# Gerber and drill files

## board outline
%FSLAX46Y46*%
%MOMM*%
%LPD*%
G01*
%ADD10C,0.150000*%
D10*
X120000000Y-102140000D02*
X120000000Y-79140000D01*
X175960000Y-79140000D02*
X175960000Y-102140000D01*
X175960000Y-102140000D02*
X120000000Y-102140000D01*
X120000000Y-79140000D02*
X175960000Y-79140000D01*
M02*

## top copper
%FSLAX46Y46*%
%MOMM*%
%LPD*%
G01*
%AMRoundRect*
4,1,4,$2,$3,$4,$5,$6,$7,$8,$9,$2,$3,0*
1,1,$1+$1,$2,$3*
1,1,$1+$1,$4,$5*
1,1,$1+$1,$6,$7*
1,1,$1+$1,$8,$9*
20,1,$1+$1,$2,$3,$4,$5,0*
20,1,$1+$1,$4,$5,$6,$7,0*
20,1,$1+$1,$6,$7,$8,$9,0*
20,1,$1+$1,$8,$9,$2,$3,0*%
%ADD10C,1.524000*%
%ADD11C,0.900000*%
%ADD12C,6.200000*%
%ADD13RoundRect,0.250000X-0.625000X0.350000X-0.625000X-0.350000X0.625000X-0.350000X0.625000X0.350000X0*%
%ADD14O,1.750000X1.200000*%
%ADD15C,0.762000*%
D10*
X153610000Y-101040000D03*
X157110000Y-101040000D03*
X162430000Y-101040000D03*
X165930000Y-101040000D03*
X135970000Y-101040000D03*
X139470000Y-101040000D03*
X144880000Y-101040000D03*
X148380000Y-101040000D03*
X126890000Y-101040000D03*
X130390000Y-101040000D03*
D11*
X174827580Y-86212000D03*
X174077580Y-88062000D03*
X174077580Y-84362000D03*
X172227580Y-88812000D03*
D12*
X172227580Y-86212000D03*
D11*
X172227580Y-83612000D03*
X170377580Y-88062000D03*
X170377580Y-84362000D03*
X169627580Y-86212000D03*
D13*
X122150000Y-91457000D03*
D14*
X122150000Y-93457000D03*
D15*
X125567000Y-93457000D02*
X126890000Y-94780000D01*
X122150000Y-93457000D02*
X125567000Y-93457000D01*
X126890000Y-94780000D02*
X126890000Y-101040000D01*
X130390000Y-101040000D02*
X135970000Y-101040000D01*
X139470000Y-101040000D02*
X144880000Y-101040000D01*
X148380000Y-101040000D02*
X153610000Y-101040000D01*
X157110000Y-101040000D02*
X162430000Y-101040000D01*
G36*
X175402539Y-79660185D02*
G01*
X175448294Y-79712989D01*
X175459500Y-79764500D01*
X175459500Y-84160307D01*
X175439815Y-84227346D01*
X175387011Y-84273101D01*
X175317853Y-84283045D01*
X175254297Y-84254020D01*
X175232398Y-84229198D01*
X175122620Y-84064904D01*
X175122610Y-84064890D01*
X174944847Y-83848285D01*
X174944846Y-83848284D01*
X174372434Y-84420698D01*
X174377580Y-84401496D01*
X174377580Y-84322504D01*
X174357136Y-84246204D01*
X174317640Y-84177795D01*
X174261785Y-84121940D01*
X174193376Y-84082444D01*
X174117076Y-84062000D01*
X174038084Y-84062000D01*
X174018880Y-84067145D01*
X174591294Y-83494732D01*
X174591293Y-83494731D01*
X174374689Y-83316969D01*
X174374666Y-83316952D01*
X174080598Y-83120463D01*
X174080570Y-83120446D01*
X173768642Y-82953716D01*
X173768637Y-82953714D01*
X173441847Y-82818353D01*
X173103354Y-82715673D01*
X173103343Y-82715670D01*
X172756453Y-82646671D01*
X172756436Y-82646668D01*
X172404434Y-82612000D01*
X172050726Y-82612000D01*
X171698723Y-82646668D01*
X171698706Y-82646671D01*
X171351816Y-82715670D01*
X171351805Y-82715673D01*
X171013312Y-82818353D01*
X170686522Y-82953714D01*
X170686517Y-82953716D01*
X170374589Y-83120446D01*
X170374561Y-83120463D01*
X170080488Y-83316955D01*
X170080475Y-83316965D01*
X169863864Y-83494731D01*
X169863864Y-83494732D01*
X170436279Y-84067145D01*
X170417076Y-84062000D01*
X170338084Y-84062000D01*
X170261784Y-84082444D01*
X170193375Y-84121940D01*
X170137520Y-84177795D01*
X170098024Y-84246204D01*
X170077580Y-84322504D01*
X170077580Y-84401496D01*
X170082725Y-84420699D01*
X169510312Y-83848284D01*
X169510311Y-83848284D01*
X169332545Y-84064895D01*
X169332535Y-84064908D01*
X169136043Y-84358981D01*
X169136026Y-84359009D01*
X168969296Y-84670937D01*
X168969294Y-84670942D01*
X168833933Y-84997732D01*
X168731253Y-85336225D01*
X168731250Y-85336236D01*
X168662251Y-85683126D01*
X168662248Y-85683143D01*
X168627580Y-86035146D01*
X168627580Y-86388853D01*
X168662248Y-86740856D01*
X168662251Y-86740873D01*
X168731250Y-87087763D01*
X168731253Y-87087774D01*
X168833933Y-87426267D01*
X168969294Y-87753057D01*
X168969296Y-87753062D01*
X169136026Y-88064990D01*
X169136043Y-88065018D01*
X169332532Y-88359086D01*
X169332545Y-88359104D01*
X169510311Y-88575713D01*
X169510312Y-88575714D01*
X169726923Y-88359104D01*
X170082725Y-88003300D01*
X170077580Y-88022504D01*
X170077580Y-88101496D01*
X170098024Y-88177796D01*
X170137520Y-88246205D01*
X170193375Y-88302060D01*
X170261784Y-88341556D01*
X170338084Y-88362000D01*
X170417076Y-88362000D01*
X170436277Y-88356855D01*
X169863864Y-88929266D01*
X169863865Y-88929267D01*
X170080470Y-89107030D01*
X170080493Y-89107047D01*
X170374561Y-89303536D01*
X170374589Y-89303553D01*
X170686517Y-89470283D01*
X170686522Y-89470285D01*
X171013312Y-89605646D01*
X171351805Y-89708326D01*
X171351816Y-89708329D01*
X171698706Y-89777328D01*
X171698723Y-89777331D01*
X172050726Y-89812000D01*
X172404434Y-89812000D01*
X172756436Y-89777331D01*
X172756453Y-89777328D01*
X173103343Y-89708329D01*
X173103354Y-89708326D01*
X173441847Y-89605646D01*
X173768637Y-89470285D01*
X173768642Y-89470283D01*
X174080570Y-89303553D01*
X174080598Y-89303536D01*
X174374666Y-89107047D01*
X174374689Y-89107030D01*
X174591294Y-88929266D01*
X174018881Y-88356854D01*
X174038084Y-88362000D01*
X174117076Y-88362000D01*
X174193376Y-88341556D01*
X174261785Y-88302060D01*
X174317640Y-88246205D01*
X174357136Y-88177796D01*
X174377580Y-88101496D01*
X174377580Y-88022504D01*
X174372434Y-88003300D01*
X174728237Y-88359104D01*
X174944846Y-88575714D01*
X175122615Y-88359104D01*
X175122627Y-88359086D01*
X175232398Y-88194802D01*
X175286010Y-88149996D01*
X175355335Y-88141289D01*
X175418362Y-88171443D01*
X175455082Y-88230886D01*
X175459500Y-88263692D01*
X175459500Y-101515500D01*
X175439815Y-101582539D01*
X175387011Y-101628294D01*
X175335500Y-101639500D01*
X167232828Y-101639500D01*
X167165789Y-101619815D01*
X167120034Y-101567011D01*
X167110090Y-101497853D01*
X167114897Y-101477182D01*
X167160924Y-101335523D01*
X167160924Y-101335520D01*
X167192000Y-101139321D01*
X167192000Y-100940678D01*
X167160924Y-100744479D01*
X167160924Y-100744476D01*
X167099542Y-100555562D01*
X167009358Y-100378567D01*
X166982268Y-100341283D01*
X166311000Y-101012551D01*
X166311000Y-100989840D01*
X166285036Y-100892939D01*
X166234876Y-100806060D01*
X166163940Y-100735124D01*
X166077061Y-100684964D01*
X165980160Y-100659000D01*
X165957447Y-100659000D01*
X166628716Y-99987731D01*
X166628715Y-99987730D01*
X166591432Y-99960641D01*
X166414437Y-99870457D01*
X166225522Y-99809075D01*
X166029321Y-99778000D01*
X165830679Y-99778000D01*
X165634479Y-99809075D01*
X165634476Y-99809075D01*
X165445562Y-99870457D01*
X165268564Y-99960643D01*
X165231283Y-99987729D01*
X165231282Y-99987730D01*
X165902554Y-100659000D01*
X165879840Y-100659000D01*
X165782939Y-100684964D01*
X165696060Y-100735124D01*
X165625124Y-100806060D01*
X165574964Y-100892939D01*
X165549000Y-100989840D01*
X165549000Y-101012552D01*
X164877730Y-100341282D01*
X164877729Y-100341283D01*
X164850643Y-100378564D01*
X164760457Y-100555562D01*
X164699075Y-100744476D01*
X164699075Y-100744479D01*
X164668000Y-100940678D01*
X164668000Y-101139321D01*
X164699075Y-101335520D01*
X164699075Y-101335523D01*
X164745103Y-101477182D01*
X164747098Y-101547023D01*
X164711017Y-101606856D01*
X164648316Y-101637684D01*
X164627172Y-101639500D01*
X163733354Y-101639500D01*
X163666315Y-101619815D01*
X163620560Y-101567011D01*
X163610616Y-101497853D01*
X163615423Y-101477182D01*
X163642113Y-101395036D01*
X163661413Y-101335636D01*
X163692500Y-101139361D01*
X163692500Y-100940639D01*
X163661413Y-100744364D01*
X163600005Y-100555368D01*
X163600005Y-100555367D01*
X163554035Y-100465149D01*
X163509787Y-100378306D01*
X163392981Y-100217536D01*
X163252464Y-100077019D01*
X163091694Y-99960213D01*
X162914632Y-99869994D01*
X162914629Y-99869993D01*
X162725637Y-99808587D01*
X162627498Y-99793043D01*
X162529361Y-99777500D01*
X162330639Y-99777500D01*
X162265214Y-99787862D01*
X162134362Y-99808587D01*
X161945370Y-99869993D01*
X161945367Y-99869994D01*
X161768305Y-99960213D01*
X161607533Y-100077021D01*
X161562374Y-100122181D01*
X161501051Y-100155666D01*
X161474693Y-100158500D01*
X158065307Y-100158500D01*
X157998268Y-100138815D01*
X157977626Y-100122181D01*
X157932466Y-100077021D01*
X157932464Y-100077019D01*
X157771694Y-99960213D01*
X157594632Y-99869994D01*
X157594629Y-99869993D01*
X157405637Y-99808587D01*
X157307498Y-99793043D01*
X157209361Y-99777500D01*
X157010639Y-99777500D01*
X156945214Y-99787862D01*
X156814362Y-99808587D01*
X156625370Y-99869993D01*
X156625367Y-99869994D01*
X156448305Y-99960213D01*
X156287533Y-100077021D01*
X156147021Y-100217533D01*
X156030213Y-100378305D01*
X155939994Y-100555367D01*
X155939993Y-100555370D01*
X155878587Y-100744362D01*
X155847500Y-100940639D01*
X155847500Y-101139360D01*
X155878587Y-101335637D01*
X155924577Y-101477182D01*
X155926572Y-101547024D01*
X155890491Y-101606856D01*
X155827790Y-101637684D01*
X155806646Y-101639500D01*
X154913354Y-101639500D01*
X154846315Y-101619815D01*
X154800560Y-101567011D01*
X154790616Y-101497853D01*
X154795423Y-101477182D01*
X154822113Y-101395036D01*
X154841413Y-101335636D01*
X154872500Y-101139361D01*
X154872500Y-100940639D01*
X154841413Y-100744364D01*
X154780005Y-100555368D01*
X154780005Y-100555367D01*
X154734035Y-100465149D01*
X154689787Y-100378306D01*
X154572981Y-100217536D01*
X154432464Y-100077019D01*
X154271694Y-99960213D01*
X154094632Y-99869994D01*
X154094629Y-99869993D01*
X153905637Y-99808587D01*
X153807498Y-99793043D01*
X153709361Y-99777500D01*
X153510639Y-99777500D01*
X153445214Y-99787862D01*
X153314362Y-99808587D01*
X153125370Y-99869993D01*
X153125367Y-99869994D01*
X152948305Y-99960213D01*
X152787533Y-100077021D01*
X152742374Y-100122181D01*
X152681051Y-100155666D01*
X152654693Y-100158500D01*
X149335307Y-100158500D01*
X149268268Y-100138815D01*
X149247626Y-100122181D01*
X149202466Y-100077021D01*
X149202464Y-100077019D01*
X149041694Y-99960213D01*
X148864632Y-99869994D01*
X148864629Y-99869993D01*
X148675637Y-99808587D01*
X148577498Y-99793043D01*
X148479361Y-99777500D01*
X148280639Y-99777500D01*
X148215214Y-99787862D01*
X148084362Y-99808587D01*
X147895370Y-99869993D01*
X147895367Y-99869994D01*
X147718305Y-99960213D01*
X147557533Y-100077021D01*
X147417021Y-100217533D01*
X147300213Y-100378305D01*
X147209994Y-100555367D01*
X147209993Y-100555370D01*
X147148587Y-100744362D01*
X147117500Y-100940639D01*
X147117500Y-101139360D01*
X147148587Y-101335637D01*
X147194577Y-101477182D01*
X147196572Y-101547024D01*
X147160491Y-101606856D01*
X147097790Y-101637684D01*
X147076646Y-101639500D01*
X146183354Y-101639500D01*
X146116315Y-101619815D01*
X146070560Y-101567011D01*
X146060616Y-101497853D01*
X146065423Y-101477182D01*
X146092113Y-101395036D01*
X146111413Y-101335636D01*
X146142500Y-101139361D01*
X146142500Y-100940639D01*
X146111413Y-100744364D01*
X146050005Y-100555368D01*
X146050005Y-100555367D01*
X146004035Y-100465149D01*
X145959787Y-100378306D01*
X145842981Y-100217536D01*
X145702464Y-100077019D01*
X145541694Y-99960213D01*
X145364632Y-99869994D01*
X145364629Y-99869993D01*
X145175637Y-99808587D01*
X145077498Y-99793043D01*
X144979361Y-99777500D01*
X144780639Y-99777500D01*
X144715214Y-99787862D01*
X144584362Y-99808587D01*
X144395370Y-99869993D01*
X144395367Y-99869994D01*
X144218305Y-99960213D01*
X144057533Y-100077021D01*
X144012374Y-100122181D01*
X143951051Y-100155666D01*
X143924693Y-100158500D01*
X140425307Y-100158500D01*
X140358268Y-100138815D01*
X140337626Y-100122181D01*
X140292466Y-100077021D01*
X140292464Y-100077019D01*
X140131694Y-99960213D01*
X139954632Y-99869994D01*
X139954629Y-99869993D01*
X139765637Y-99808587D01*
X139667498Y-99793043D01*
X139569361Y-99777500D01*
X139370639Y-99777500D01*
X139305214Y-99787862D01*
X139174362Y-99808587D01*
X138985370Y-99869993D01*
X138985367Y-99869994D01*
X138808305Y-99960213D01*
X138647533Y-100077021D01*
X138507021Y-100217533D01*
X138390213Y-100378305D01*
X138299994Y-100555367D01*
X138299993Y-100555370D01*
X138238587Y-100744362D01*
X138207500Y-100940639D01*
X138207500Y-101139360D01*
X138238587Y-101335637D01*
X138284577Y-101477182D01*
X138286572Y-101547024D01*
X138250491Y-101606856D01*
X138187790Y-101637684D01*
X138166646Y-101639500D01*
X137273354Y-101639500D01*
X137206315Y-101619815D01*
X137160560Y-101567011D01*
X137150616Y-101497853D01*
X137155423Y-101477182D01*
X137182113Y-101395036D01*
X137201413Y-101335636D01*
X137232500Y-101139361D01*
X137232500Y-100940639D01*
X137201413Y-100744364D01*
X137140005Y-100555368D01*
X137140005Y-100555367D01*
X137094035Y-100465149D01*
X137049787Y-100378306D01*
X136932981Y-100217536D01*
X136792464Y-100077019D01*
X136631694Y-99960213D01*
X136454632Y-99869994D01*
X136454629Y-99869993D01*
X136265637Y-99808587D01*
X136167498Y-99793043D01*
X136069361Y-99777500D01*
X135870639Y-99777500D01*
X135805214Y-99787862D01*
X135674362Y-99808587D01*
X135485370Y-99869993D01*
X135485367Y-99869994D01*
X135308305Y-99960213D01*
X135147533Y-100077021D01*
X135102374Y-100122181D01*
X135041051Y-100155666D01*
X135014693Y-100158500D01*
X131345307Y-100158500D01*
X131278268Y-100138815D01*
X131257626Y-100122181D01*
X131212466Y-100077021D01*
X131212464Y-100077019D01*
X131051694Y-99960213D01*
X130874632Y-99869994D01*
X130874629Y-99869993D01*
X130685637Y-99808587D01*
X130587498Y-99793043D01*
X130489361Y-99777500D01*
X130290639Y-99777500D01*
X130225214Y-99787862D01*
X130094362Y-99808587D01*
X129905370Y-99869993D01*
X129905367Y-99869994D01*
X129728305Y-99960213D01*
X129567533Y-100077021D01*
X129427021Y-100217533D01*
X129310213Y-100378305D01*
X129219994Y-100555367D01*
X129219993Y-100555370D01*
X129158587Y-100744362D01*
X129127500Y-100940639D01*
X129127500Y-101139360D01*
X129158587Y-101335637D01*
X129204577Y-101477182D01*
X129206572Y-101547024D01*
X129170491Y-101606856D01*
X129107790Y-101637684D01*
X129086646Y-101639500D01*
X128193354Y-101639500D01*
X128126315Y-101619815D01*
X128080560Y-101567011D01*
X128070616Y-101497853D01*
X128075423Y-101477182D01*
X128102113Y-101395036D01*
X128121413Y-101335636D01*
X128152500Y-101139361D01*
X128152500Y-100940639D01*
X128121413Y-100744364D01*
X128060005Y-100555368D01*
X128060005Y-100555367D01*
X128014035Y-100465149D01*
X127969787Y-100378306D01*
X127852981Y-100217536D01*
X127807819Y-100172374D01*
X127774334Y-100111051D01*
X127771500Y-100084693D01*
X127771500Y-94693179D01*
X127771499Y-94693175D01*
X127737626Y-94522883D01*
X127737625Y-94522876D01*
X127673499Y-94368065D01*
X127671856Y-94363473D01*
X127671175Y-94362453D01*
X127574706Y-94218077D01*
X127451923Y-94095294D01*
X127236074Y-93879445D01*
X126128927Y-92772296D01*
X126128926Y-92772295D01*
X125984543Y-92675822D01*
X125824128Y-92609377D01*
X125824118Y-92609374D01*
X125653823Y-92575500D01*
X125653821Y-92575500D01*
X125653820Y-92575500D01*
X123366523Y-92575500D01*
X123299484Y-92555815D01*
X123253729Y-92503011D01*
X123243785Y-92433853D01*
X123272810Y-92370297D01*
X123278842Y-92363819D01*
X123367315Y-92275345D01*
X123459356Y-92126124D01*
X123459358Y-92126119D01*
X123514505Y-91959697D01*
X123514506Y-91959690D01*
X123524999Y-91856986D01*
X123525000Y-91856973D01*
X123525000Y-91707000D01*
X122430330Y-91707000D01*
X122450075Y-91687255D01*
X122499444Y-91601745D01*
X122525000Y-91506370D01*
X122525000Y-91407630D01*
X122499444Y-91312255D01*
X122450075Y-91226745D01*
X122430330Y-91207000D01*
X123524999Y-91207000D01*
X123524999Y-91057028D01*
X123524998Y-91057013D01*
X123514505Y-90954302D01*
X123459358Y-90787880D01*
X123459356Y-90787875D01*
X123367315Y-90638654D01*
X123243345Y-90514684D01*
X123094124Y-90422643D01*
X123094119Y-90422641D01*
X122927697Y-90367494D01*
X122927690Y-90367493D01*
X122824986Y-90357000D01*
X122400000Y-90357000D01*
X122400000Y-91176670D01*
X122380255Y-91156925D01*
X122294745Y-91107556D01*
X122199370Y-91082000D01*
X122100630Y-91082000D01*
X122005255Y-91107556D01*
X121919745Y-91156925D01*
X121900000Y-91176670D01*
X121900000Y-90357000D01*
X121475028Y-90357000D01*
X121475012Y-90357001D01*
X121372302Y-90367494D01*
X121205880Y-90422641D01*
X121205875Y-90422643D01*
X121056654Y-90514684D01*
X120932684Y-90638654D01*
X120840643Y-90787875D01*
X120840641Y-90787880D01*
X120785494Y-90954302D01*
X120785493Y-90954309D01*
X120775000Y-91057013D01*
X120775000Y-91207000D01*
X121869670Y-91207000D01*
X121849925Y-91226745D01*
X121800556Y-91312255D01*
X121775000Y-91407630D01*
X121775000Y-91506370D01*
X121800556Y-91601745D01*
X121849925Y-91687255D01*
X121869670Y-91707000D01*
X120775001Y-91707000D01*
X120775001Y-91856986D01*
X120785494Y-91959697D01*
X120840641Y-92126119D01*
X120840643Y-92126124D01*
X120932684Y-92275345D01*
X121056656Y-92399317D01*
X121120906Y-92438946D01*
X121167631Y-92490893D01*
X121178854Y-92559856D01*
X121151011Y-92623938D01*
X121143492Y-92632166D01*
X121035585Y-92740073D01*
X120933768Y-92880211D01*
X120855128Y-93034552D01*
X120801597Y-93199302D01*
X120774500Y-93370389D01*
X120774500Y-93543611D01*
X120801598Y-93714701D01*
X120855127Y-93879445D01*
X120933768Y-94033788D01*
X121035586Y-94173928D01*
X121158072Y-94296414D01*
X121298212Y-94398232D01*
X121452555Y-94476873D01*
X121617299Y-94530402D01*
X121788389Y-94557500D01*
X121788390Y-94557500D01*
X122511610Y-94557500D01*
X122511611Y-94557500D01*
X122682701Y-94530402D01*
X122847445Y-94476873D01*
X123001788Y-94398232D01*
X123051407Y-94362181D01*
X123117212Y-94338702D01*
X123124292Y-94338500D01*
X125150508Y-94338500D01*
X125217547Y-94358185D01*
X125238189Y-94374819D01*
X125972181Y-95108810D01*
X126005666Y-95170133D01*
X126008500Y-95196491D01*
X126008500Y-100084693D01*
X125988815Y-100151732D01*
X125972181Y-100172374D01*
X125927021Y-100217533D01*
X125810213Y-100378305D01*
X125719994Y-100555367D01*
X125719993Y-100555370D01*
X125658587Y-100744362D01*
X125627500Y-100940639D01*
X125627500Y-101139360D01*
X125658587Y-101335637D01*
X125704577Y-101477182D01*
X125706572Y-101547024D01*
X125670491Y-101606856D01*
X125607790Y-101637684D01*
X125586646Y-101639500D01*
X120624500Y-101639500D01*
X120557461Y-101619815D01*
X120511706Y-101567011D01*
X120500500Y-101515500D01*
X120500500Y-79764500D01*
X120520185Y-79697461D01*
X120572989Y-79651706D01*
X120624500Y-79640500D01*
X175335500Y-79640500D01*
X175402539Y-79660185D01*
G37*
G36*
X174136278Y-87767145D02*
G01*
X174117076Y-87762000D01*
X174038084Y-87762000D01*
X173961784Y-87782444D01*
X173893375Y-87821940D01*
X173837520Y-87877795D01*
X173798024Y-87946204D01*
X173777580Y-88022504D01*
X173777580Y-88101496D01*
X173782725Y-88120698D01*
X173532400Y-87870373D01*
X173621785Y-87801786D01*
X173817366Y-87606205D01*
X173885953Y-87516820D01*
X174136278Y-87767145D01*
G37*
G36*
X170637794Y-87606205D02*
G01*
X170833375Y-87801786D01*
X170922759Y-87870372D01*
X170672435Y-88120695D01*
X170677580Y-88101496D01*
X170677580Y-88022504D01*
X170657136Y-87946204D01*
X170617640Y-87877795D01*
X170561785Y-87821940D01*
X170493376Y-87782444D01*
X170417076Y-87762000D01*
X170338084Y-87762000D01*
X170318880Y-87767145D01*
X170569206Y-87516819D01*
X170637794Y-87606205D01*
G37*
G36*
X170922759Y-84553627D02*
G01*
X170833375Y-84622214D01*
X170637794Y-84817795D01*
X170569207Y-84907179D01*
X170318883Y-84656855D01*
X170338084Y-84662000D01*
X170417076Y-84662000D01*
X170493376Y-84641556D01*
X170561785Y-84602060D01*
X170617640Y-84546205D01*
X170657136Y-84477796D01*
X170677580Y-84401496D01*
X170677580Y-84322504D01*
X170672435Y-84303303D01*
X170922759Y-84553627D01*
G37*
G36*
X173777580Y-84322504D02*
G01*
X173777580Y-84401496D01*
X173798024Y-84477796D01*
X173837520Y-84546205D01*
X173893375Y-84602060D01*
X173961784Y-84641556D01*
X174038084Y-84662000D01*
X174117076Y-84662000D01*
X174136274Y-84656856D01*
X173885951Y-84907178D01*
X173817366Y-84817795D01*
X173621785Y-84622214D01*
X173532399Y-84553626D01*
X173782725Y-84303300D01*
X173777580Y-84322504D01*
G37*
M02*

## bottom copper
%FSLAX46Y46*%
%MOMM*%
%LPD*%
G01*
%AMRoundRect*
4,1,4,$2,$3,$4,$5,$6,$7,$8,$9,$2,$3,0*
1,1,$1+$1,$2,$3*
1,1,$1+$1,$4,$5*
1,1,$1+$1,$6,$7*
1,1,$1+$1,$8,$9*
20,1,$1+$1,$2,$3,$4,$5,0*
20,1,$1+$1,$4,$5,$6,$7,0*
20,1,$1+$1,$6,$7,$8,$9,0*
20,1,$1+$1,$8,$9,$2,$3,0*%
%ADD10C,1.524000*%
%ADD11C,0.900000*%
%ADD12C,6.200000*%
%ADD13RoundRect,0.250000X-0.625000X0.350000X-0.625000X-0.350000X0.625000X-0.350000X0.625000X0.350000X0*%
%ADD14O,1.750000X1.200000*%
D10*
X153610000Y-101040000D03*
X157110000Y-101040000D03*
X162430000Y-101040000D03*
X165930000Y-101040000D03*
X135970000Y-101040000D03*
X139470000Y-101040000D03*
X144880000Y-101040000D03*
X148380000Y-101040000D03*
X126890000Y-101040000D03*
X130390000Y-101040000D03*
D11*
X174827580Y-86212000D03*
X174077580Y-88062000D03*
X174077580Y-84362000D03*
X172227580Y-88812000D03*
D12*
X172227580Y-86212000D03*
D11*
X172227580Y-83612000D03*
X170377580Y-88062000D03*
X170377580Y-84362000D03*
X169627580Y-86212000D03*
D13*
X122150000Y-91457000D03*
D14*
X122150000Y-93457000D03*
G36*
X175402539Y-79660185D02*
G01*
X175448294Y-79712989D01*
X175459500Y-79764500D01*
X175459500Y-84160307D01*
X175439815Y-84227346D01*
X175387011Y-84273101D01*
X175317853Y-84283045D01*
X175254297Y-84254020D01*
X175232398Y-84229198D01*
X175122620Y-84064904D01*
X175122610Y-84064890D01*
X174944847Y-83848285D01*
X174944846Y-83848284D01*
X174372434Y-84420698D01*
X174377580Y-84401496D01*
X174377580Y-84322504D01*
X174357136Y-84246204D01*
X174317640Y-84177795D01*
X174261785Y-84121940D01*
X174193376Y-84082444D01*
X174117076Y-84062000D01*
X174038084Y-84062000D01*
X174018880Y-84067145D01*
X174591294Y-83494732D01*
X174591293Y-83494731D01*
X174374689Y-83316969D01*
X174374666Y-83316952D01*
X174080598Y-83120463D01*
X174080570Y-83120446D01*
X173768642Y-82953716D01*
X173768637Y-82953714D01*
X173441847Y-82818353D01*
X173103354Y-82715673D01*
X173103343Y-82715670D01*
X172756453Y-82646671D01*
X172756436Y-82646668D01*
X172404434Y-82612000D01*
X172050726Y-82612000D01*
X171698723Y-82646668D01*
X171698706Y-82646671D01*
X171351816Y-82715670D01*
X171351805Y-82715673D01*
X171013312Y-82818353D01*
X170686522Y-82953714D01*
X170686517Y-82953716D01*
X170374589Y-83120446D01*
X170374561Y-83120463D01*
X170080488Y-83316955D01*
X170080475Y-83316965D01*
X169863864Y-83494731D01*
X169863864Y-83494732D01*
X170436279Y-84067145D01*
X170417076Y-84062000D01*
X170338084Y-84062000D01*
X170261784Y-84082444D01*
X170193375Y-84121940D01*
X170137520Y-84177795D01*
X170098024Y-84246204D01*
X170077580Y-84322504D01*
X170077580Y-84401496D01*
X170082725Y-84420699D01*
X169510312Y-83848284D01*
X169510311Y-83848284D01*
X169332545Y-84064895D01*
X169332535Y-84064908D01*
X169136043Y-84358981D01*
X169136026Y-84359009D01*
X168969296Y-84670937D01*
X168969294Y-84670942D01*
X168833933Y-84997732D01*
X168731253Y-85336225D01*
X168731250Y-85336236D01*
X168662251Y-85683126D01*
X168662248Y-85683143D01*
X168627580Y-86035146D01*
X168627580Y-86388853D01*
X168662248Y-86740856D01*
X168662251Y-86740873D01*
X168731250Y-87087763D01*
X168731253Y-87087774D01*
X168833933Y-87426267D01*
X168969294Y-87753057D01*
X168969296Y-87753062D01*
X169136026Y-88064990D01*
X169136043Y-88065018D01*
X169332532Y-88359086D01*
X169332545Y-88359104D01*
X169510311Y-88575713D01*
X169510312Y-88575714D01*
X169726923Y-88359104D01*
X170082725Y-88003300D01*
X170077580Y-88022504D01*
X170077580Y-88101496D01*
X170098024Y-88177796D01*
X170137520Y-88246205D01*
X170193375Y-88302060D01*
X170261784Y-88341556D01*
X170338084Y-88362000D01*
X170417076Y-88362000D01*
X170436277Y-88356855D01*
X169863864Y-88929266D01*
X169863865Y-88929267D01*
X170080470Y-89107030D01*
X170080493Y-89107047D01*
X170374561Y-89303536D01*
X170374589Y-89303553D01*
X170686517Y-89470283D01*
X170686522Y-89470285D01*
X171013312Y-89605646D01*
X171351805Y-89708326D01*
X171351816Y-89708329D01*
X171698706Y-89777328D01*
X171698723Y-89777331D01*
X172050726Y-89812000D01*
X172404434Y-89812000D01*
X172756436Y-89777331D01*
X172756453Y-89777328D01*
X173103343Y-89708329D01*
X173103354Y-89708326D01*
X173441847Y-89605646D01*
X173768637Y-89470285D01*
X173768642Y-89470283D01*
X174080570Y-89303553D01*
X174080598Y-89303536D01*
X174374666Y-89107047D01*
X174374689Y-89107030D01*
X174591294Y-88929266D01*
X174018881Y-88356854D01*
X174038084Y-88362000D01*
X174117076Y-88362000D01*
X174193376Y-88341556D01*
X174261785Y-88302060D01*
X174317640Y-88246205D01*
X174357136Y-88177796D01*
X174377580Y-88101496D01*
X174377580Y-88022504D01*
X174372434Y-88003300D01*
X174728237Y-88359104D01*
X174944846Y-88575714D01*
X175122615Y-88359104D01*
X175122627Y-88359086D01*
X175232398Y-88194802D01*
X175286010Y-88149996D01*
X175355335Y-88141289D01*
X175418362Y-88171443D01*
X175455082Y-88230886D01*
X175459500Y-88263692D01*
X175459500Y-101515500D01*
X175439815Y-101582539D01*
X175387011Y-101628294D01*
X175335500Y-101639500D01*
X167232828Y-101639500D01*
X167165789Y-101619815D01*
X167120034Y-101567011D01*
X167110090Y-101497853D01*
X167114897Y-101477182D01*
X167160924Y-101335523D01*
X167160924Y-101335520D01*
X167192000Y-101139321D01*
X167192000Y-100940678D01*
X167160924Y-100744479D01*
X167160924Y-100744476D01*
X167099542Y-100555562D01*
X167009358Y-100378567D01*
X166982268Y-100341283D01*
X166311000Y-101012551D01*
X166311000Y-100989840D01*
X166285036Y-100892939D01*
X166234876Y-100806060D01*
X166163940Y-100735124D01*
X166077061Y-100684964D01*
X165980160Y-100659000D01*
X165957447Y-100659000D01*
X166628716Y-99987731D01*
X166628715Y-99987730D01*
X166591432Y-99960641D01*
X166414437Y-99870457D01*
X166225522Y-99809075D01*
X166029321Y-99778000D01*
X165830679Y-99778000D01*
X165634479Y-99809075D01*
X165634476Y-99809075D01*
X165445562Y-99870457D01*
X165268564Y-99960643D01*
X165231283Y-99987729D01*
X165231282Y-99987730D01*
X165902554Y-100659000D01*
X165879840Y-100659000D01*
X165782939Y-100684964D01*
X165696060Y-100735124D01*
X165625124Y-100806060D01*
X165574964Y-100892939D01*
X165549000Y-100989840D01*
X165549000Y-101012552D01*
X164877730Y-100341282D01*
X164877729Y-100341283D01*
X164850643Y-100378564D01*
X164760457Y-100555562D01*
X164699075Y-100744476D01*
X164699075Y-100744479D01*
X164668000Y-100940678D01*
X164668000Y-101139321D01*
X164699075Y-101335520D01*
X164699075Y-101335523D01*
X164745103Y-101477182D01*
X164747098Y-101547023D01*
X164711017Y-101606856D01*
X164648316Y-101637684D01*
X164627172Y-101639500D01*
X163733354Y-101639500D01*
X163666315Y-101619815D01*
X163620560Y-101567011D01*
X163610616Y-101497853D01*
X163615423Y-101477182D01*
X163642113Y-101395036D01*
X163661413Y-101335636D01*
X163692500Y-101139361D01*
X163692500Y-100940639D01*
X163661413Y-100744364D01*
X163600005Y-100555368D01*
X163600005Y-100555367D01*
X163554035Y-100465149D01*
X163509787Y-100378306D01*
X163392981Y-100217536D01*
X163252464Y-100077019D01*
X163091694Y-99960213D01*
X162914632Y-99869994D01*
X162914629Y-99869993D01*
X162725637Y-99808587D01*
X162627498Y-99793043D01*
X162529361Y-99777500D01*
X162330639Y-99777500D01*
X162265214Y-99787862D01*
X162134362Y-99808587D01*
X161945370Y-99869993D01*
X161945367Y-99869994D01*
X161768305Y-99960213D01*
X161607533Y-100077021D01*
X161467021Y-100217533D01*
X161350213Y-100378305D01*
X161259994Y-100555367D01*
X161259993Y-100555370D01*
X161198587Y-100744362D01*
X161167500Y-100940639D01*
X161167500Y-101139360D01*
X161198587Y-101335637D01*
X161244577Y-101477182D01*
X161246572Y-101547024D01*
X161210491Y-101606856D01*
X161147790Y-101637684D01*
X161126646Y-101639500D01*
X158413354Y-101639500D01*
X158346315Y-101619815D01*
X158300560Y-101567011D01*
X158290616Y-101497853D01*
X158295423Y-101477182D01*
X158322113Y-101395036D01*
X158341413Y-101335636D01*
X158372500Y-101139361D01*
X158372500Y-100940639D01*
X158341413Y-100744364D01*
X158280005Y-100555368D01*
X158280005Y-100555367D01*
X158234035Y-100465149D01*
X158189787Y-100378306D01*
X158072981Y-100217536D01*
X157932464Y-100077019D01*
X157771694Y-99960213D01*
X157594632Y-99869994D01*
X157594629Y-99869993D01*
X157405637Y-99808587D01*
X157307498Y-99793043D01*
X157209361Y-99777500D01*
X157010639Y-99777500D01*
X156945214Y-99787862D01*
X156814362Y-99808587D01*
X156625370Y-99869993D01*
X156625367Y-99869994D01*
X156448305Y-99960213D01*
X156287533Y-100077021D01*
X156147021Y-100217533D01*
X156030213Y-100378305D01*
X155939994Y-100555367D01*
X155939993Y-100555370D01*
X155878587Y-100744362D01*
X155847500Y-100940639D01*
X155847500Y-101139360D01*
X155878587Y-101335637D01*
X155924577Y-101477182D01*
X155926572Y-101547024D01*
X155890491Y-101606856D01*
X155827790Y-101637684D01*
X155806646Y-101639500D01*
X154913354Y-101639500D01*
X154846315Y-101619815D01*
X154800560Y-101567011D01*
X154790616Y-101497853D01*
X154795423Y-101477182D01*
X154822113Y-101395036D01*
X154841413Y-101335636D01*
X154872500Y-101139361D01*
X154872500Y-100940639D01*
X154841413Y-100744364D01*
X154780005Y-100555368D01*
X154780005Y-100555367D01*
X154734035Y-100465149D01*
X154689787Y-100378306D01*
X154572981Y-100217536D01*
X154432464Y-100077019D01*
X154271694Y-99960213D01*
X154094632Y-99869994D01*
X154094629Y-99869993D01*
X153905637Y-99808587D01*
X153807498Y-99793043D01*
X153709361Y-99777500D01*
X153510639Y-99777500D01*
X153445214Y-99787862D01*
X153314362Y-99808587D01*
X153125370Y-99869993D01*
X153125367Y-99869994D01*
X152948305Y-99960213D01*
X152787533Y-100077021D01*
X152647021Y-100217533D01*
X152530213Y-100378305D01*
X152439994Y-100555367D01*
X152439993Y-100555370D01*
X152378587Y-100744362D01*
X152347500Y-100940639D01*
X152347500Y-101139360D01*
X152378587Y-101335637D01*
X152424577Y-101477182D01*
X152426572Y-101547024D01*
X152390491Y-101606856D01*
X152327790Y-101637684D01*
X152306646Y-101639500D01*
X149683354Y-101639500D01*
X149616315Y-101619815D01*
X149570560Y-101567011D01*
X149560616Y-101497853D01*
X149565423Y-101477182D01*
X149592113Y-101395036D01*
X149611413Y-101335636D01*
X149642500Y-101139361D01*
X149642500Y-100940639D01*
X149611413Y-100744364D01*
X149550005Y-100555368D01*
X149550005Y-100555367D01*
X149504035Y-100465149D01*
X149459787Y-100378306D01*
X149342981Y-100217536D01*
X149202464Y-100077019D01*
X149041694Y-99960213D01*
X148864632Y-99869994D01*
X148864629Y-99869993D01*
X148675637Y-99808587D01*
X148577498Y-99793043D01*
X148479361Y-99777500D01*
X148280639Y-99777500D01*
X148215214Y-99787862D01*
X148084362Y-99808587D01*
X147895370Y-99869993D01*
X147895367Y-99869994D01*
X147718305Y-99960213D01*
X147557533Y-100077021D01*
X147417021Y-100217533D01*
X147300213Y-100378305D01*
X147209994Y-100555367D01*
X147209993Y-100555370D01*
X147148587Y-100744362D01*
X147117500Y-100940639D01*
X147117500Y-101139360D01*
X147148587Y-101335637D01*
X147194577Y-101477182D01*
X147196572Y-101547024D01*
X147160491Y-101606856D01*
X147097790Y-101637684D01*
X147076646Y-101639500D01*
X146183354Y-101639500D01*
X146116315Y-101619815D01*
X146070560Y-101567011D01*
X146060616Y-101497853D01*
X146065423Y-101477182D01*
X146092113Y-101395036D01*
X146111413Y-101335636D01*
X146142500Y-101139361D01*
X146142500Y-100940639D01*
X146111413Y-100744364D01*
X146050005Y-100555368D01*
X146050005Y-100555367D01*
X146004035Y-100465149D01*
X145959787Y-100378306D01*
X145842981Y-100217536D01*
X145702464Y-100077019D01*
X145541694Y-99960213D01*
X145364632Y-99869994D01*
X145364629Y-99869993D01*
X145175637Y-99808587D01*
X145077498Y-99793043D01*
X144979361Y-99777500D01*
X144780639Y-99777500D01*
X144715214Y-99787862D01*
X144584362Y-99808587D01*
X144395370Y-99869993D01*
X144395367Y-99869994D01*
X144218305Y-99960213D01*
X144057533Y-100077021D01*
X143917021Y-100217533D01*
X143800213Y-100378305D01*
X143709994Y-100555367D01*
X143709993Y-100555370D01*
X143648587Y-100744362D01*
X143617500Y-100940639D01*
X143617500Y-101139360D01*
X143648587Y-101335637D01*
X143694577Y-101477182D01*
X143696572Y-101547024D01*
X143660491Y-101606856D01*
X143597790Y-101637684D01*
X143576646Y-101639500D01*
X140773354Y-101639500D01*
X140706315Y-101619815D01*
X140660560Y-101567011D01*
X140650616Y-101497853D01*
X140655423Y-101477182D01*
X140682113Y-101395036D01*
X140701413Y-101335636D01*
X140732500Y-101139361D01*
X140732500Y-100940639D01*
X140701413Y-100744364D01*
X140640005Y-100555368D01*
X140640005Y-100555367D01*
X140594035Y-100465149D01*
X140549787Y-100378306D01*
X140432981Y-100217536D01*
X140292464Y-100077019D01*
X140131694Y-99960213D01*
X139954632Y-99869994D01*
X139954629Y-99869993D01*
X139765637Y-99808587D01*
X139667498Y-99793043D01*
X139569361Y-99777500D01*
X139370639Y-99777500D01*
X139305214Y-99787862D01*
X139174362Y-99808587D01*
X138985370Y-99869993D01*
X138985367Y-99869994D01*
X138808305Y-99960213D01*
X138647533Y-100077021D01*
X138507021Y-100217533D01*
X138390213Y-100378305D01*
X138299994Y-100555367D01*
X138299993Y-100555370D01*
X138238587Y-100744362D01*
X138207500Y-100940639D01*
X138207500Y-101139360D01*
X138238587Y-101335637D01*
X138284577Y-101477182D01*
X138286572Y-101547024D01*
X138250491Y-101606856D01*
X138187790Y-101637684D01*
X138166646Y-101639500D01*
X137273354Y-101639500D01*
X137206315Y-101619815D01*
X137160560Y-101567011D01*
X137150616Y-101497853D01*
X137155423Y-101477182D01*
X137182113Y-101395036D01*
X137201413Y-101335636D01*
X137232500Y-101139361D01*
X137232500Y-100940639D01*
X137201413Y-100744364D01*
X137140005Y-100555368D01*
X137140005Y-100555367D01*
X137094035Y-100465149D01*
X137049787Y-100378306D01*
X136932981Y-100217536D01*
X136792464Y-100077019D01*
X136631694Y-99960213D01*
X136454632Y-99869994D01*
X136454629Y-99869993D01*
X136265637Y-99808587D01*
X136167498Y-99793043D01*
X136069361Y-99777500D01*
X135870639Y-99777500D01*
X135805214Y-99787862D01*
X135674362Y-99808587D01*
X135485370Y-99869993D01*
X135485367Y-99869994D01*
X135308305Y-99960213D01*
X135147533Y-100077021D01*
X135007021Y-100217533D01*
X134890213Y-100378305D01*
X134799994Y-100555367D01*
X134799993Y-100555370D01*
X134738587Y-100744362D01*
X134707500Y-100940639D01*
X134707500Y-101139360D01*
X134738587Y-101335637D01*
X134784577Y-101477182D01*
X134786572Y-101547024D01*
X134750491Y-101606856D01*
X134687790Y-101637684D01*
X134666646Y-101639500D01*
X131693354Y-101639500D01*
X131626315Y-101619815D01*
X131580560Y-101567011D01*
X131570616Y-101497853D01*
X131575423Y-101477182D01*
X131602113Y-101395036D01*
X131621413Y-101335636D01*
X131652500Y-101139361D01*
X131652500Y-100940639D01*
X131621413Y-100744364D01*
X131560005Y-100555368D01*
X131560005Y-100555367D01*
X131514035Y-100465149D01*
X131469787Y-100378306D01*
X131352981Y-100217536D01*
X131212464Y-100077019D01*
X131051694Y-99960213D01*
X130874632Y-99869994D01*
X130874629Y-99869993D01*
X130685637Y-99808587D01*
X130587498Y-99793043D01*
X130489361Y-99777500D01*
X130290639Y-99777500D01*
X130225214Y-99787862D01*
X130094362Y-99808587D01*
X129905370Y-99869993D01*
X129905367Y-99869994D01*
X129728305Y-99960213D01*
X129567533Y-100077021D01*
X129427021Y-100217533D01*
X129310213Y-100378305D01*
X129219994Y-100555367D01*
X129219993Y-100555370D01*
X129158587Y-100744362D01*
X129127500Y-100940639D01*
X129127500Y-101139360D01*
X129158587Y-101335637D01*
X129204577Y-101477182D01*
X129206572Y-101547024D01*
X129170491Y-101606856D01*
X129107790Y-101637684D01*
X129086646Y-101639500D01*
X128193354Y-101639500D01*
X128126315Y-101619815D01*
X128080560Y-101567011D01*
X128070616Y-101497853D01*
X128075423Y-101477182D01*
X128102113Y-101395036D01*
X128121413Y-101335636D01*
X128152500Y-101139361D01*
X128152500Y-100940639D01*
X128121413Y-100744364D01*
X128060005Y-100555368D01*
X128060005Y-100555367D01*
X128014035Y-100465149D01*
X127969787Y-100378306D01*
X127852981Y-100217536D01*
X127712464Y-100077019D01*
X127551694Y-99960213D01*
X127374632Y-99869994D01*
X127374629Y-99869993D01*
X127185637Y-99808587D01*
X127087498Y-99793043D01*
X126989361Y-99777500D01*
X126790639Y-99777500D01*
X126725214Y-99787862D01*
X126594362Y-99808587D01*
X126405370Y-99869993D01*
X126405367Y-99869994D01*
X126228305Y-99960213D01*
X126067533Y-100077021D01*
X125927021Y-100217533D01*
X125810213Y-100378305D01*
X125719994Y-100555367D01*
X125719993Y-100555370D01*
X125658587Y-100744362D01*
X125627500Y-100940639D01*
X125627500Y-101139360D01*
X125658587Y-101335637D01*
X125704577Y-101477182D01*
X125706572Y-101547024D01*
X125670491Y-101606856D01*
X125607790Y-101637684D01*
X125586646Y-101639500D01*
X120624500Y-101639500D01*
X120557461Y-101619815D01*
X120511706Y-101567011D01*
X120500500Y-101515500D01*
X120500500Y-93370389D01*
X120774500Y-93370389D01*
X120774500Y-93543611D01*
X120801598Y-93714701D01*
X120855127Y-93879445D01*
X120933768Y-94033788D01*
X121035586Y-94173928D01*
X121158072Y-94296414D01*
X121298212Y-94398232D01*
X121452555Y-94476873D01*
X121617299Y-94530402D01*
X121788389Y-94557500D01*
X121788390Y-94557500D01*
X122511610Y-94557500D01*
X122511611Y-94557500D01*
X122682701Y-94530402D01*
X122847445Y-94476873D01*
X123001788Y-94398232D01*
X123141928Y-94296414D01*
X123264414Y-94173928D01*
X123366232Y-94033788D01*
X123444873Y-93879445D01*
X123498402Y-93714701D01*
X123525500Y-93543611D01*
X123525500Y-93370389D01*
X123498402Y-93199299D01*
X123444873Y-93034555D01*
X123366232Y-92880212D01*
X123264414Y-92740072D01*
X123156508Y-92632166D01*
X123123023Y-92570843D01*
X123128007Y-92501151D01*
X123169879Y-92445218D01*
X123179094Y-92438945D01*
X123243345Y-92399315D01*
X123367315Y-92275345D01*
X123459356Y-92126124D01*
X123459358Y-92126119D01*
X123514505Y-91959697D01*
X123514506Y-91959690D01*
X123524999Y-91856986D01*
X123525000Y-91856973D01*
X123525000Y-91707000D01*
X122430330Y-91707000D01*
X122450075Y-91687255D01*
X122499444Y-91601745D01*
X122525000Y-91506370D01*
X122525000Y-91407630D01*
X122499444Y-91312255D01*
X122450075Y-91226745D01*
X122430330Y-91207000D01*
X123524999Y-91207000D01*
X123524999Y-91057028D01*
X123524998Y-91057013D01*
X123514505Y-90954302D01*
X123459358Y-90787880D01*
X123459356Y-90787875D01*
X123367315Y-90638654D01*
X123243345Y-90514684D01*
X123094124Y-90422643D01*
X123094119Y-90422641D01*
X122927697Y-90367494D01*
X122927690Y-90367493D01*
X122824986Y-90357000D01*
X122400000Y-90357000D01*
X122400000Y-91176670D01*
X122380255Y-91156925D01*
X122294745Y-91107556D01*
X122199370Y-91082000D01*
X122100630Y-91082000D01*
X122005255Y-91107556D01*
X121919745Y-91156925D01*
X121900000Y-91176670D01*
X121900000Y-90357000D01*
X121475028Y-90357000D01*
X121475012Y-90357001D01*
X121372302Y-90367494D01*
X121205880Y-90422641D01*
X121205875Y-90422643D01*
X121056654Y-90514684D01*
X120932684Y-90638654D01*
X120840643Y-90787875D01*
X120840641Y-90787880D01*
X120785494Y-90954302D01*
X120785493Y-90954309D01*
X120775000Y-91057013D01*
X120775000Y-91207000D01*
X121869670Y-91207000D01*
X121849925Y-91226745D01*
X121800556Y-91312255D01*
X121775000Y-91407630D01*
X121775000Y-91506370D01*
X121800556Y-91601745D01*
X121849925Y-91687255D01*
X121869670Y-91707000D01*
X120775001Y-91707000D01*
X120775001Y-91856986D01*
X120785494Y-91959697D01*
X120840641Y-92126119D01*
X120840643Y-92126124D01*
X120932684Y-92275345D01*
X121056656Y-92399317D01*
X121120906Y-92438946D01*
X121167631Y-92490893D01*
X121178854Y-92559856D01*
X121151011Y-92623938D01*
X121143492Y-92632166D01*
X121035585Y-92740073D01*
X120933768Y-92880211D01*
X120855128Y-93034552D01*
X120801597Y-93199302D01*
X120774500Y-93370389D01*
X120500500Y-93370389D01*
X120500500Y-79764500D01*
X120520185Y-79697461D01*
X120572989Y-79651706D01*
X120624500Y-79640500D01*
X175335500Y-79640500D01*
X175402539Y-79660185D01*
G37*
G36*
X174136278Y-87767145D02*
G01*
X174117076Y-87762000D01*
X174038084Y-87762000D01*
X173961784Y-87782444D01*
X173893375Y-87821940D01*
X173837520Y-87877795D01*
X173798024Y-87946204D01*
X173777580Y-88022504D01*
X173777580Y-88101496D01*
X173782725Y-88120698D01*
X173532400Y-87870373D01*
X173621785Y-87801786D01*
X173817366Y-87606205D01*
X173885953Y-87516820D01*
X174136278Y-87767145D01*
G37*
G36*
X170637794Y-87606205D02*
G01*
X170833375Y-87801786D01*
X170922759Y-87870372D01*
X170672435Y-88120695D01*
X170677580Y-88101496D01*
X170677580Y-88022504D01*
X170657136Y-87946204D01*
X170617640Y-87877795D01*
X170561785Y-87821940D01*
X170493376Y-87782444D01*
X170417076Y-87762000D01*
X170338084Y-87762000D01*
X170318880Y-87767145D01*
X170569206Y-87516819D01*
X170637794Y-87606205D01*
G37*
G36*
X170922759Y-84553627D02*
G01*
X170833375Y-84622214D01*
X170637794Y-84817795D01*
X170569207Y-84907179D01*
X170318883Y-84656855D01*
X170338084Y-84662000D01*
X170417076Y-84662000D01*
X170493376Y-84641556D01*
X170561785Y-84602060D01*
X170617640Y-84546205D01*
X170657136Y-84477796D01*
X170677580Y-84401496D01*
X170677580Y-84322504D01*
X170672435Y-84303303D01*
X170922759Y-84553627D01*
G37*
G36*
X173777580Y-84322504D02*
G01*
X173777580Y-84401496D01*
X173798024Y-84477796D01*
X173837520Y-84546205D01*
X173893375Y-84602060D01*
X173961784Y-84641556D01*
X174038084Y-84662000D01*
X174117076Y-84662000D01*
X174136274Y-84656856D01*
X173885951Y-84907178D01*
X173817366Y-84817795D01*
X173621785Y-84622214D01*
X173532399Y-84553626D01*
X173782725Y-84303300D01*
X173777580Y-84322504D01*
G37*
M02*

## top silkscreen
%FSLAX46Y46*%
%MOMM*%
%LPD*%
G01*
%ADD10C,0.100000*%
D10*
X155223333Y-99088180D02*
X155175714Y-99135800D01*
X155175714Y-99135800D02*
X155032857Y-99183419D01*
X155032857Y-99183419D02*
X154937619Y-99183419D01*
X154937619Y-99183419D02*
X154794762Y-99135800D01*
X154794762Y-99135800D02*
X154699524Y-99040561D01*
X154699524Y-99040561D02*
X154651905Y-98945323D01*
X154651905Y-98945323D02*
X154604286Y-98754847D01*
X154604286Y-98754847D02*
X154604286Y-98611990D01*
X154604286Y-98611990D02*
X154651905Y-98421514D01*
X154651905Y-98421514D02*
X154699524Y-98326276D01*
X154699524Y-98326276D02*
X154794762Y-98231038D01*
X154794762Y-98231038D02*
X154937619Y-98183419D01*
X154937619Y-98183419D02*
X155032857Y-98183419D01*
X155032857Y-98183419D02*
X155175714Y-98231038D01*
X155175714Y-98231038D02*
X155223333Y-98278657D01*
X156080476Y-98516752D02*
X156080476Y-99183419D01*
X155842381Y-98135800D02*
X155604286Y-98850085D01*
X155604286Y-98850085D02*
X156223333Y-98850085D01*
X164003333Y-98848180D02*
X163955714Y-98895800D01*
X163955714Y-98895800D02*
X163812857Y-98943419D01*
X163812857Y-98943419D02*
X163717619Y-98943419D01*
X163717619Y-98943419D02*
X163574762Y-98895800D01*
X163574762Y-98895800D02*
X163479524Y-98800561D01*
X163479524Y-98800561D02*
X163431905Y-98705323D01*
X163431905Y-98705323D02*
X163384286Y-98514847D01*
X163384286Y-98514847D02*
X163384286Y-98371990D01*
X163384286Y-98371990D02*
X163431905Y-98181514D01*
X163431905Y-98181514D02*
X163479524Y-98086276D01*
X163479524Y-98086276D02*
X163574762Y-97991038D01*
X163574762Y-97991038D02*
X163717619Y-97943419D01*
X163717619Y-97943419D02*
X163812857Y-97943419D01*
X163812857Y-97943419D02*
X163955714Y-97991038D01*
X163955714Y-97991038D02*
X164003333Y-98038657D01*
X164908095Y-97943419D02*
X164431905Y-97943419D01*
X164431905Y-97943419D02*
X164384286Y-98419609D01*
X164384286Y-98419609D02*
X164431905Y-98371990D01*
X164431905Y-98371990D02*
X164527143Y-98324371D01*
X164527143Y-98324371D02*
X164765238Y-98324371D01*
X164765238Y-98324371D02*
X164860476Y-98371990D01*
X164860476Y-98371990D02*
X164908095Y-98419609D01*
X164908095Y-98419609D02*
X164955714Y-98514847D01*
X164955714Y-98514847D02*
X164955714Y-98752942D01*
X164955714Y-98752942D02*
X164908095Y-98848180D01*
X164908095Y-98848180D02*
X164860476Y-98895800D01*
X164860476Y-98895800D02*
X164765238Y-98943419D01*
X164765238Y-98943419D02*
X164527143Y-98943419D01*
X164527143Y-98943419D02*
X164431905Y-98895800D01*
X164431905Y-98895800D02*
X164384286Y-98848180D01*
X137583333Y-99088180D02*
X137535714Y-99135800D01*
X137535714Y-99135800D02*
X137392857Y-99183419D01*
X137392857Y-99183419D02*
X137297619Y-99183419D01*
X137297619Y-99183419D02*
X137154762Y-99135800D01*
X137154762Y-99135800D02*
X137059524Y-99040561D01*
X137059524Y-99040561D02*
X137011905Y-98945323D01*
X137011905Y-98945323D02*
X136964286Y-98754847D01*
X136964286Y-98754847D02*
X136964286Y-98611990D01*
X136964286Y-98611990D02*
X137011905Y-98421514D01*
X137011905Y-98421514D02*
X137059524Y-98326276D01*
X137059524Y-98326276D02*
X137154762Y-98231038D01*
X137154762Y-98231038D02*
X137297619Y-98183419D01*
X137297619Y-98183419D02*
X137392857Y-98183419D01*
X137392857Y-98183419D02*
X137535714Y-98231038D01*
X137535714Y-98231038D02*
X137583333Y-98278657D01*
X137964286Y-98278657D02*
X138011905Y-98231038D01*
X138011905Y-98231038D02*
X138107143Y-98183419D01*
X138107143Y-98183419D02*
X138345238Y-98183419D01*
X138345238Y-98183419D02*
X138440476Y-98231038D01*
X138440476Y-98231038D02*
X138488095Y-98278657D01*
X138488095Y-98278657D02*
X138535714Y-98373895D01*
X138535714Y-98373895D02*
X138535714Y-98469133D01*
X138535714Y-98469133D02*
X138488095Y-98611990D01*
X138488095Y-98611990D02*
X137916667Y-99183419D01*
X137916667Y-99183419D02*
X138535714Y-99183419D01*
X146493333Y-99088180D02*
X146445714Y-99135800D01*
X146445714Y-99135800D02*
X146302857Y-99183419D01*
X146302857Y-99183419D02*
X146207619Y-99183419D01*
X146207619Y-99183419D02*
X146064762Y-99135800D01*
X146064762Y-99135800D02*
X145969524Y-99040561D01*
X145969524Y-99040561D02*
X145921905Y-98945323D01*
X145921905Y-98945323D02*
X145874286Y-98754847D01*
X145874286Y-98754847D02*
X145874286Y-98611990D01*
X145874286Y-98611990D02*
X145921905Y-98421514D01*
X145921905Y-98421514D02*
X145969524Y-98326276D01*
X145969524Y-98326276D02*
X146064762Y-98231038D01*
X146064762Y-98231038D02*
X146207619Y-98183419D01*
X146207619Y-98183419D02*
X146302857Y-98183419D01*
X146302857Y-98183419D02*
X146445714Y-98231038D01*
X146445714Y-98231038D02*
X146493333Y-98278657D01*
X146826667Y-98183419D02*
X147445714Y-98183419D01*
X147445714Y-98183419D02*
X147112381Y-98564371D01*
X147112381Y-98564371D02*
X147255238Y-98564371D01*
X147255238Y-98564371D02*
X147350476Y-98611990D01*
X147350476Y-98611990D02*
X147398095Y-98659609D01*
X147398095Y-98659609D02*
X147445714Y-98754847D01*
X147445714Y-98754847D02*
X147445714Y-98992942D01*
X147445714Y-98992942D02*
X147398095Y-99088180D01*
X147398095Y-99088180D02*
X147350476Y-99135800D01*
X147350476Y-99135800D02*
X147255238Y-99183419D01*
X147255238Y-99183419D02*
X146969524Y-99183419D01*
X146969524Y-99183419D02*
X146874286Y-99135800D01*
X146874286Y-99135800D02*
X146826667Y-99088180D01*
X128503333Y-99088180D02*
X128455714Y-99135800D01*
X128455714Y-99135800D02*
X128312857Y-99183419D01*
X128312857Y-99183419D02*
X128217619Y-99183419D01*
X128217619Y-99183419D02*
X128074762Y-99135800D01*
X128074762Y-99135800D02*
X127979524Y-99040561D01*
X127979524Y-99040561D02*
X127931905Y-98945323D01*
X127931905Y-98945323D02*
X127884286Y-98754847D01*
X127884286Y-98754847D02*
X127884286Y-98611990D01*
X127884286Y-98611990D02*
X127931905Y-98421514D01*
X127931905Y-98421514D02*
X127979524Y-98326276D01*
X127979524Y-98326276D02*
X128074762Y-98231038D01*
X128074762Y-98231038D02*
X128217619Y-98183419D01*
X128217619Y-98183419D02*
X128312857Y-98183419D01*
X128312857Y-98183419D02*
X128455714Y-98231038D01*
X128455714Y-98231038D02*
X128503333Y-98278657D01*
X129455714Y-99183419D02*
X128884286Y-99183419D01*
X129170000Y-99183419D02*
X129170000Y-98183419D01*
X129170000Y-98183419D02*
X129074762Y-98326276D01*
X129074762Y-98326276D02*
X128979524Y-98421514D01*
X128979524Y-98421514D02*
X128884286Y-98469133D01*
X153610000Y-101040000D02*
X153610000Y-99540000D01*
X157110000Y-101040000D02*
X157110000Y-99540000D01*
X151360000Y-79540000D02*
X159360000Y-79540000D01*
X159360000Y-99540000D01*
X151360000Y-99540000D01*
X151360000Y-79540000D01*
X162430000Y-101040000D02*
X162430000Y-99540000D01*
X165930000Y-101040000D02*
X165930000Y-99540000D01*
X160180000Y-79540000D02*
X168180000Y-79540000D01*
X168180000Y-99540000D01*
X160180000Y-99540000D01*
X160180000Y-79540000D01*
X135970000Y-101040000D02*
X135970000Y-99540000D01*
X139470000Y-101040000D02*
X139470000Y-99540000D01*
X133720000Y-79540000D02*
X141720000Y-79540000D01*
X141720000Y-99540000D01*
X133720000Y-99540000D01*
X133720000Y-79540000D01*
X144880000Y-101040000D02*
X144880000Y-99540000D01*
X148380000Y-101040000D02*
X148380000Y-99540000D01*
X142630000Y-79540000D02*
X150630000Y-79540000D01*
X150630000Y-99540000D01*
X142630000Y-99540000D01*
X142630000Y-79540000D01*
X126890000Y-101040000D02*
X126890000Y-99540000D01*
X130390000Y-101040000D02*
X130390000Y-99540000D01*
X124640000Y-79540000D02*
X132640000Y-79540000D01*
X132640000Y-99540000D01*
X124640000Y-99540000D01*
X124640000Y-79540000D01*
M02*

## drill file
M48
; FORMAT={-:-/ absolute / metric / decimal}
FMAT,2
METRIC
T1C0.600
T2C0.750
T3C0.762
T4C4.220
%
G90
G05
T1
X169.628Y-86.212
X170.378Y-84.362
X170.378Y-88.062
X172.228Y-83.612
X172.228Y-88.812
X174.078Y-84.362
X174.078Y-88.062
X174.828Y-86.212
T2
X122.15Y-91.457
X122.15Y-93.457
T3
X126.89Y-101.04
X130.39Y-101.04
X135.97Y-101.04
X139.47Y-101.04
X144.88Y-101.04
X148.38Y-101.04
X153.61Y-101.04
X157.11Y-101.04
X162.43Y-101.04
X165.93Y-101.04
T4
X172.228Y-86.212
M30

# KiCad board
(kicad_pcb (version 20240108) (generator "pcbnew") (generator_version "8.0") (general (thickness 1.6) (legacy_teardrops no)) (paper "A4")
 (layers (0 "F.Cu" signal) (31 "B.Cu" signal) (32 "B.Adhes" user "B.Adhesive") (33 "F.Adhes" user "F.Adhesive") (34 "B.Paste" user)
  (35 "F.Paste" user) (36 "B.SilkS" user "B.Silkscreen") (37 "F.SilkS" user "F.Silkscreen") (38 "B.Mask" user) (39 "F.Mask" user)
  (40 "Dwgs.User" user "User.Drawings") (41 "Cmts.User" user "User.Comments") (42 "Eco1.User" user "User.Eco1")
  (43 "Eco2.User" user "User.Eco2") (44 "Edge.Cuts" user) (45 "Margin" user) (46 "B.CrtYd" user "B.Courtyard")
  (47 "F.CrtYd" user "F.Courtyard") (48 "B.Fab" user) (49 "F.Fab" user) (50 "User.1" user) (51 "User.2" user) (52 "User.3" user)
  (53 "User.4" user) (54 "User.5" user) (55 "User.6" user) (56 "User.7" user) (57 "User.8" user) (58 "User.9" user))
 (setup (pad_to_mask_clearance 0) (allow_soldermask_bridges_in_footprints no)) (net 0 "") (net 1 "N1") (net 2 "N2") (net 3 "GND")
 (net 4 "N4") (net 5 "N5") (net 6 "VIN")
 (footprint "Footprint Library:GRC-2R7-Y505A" (layer "F.Cu") (at 153.61 101.04)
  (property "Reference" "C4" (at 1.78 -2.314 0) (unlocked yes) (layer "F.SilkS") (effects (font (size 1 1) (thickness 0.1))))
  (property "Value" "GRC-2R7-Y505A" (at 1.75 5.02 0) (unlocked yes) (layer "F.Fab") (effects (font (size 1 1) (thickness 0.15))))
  (fp_line (start 0 0) (end 0 -1.5) (stroke (width 0.1) (type default)) (layer "F.SilkS"))
  (fp_line (start 3.5 0) (end 3.5 -1.5) (stroke (width 0.1) (type default)) (layer "F.SilkS"))
  (fp_rect (start -2.25 -21.5) (end 5.75 -1.5) (stroke (width 0.1) (type default)) (fill none) (layer "F.SilkS"))
  (pad "1" thru_hole circle (at 0 0) (size 1.524 1.524) (drill 0.762) (layers "*.Cu" "*.Mask") (remove_unused_layers no) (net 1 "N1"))
  (pad "2" thru_hole circle (at 3.5 0) (size 1.524 1.524) (drill 0.762) (layers "*.Cu" "*.Mask") (remove_unused_layers no) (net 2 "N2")))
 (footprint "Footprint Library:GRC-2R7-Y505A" (layer "F.Cu") (at 162.43 101.04)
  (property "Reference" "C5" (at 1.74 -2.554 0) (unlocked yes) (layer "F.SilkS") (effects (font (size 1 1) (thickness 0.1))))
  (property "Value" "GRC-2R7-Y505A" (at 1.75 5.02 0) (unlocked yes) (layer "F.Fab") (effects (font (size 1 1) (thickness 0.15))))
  (fp_line (start 0 0) (end 0 -1.5) (stroke (width 0.1) (type default)) (layer "F.SilkS"))
  (fp_line (start 3.5 0) (end 3.5 -1.5) (stroke (width 0.1) (type default)) (layer "F.SilkS"))
  (fp_rect (start -2.25 -21.5) (end 5.75 -1.5) (stroke (width 0.1) (type default)) (fill none) (layer "F.SilkS"))
  (pad "1" thru_hole circle (at 0 0) (size 1.524 1.524) (drill 0.762) (layers "*.Cu" "*.Mask") (remove_unused_layers no) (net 2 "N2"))
  (pad "2" thru_hole circle (at 3.5 0) (size 1.524 1.524) (drill 0.762) (layers "*.Cu" "*.Mask") (remove_unused_layers no) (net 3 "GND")))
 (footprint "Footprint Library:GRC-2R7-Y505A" (layer "F.Cu") (at 135.97 101.04)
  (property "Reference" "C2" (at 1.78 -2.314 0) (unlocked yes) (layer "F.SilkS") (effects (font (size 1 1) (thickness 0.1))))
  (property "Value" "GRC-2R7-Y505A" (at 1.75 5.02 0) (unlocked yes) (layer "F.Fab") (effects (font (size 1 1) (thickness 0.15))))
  (fp_line (start 0 0) (end 0 -1.5) (stroke (width 0.1) (type default)) (layer "F.SilkS"))
  (fp_line (start 3.5 0) (end 3.5 -1.5) (stroke (width 0.1) (type default)) (layer "F.SilkS"))
  (fp_rect (start -2.25 -21.5) (end 5.75 -1.5) (stroke (width 0.1) (type default)) (fill none) (layer "F.SilkS"))
  (pad "1" thru_hole circle (at 0 0) (size 1.524 1.524) (drill 0.762) (layers "*.Cu" "*.Mask") (remove_unused_layers no) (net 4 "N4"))
  (pad "2" thru_hole circle (at 3.5 0) (size 1.524 1.524) (drill 0.762) (layers "*.Cu" "*.Mask") (remove_unused_layers no) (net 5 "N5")))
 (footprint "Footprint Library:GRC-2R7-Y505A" (layer "F.Cu") (at 144.88 101.04)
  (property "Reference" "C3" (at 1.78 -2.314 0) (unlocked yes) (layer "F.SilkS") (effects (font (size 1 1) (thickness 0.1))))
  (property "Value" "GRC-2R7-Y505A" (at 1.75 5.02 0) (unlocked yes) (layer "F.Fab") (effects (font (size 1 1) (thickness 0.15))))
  (fp_line (start 0 0) (end 0 -1.5) (stroke (width 0.1) (type default)) (layer "F.SilkS"))
  (fp_line (start 3.5 0) (end 3.5 -1.5) (stroke (width 0.1) (type default)) (layer "F.SilkS"))
  (fp_rect (start -2.25 -21.5) (end 5.75 -1.5) (stroke (width 0.1) (type default)) (fill none) (layer "F.SilkS"))
  (pad "1" thru_hole circle (at 0 0) (size 1.524 1.524) (drill 0.762) (layers "*.Cu" "*.Mask") (remove_unused_layers no) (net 5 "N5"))
  (pad "2" thru_hole circle (at 3.5 0) (size 1.524 1.524) (drill 0.762) (layers "*.Cu" "*.Mask") (remove_unused_layers no) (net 1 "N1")))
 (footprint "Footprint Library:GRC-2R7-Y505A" (layer "F.Cu") (at 126.89 101.04)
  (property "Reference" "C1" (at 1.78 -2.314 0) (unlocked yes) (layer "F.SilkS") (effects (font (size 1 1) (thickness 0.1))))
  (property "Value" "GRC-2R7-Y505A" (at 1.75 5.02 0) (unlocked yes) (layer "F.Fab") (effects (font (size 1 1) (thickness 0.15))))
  (fp_line (start 0 0) (end 0 -1.5) (stroke (width 0.1) (type default)) (layer "F.SilkS"))
  (fp_line (start 3.5 0) (end 3.5 -1.5) (stroke (width 0.1) (type default)) (layer "F.SilkS"))
  (fp_rect (start -2.25 -21.5) (end 5.75 -1.5) (stroke (width 0.1) (type default)) (fill none) (layer "F.SilkS"))
  (pad "1" thru_hole circle (at 0 0) (size 1.524 1.524) (drill 0.762) (layers "*.Cu" "*.Mask") (remove_unused_layers no) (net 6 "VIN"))
  (pad "2" thru_hole circle (at 3.5 0) (size 1.524 1.524) (drill 0.762) (layers "*.Cu" "*.Mask") (remove_unused_layers no) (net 4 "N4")))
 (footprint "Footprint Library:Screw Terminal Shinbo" (layer "B.Cu") (at 172.22758 86.212 180)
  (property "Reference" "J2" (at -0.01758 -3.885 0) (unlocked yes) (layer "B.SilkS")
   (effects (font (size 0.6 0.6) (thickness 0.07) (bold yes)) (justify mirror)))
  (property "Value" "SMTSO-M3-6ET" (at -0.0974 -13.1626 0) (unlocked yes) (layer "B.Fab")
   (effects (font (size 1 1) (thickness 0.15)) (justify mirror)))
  (pad "1" thru_hole circle (at -2.6 0 180) (size 0.9 0.9) (drill 0.6) (layers "*.Cu" "*.Mask") (remove_unused_layers no) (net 3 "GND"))
  (pad "1" thru_hole circle (at -1.85 -1.85 180) (size 0.9 0.9) (drill 0.6) (layers "*.Cu" "*.Mask") (remove_unused_layers no) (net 3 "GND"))
  (pad "1" thru_hole circle (at -1.85 1.85 180) (size 0.9 0.9) (drill 0.6) (layers "*.Cu" "*.Mask") (remove_unused_layers no) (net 3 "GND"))
  (pad "1" thru_hole circle (at 0 -2.6 180) (size 0.9 0.9) (drill 0.6) (layers "*.Cu" "*.Mask") (remove_unused_layers no) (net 3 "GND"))
  (pad "1" thru_hole circle (at 0 0 180) (size 6.2 6.2) (drill 4.22) (layers "*.Cu" "*.Mask") (remove_unused_layers no) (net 3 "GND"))
  (pad "1" thru_hole circle (at 0 2.6 180) (size 0.9 0.9) (drill 0.6) (layers "*.Cu" "*.Mask") (remove_unused_layers no) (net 3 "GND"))
  (pad "1" thru_hole circle (at 1.85 -1.85 180) (size 0.9 0.9) (drill 0.6) (layers "*.Cu" "*.Mask") (remove_unused_layers no) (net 3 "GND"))
  (pad "1" thru_hole circle (at 1.85 1.85 180) (size 0.9 0.9) (drill 0.6) (layers "*.Cu" "*.Mask") (remove_unused_layers no) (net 3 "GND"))
  (pad "1" thru_hole circle (at 2.6 0 180) (size 0.9 0.9) (drill 0.6) (layers "*.Cu" "*.Mask") (remove_unused_layers no) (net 3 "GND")))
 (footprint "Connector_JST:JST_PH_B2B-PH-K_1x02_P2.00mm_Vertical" (layer "B.Cu") (at 122.15 91.457 -90)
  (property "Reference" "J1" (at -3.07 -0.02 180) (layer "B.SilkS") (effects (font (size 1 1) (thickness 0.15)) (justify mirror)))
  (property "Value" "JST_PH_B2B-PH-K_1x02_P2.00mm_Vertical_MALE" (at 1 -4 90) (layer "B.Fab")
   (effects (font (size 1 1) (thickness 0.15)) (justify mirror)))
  (pad "1" thru_hole roundrect (at 0 0 270) (size 1.2 1.75) (drill 0.75) (layers "*.Cu" "*.Mask") (remove_unused_layers no)
   (roundrect_rratio 0.2083333333) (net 3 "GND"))
  (pad "2" thru_hole oval (at 2 0 270) (size 1.2 1.75) (drill 0.75) (layers "*.Cu" "*.Mask") (remove_unused_layers no) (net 6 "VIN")))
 (gr_line (start 120 102.14) (end 120 79.14) (stroke (width 0.15) (type default)) (layer "Edge.Cuts"))
 (gr_line (start 175.96 79.14) (end 175.96 102.14) (stroke (width 0.15) (type default)) (layer "Edge.Cuts"))
 (gr_line (start 175.96 102.14) (end 120 102.14) (stroke (width 0.15) (type default)) (layer "Edge.Cuts"))
 (gr_line (start 120 79.14) (end 175.96 79.14) (stroke (width 0.15) (type default)) (layer "Edge.Cuts"))
 (segment (start 125.567 93.457) (end 126.89 94.78) (width 0.762) (layer "F.Cu") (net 6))
 (segment (start 122.15 93.457) (end 125.567 93.457) (width 0.762) (layer "F.Cu") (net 6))
 (segment (start 126.89 94.78) (end 126.89 101.04) (width 0.762) (layer "F.Cu") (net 6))
 (segment (start 130.39 101.04) (end 135.97 101.04) (width 0.762) (layer "F.Cu") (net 4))
 (segment (start 139.47 101.04) (end 144.88 101.04) (width 0.762) (layer "F.Cu") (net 5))
 (segment (start 148.38 101.04) (end 153.61 101.04) (width 0.762) (layer "F.Cu") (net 1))
 (segment (start 157.11 101.04) (end 162.43 101.04) (width 0.762) (layer "F.Cu") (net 2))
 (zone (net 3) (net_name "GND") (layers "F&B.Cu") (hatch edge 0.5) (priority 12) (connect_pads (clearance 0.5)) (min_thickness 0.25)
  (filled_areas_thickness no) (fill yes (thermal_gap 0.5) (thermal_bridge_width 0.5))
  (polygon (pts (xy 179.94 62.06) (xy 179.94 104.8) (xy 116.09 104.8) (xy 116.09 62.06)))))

